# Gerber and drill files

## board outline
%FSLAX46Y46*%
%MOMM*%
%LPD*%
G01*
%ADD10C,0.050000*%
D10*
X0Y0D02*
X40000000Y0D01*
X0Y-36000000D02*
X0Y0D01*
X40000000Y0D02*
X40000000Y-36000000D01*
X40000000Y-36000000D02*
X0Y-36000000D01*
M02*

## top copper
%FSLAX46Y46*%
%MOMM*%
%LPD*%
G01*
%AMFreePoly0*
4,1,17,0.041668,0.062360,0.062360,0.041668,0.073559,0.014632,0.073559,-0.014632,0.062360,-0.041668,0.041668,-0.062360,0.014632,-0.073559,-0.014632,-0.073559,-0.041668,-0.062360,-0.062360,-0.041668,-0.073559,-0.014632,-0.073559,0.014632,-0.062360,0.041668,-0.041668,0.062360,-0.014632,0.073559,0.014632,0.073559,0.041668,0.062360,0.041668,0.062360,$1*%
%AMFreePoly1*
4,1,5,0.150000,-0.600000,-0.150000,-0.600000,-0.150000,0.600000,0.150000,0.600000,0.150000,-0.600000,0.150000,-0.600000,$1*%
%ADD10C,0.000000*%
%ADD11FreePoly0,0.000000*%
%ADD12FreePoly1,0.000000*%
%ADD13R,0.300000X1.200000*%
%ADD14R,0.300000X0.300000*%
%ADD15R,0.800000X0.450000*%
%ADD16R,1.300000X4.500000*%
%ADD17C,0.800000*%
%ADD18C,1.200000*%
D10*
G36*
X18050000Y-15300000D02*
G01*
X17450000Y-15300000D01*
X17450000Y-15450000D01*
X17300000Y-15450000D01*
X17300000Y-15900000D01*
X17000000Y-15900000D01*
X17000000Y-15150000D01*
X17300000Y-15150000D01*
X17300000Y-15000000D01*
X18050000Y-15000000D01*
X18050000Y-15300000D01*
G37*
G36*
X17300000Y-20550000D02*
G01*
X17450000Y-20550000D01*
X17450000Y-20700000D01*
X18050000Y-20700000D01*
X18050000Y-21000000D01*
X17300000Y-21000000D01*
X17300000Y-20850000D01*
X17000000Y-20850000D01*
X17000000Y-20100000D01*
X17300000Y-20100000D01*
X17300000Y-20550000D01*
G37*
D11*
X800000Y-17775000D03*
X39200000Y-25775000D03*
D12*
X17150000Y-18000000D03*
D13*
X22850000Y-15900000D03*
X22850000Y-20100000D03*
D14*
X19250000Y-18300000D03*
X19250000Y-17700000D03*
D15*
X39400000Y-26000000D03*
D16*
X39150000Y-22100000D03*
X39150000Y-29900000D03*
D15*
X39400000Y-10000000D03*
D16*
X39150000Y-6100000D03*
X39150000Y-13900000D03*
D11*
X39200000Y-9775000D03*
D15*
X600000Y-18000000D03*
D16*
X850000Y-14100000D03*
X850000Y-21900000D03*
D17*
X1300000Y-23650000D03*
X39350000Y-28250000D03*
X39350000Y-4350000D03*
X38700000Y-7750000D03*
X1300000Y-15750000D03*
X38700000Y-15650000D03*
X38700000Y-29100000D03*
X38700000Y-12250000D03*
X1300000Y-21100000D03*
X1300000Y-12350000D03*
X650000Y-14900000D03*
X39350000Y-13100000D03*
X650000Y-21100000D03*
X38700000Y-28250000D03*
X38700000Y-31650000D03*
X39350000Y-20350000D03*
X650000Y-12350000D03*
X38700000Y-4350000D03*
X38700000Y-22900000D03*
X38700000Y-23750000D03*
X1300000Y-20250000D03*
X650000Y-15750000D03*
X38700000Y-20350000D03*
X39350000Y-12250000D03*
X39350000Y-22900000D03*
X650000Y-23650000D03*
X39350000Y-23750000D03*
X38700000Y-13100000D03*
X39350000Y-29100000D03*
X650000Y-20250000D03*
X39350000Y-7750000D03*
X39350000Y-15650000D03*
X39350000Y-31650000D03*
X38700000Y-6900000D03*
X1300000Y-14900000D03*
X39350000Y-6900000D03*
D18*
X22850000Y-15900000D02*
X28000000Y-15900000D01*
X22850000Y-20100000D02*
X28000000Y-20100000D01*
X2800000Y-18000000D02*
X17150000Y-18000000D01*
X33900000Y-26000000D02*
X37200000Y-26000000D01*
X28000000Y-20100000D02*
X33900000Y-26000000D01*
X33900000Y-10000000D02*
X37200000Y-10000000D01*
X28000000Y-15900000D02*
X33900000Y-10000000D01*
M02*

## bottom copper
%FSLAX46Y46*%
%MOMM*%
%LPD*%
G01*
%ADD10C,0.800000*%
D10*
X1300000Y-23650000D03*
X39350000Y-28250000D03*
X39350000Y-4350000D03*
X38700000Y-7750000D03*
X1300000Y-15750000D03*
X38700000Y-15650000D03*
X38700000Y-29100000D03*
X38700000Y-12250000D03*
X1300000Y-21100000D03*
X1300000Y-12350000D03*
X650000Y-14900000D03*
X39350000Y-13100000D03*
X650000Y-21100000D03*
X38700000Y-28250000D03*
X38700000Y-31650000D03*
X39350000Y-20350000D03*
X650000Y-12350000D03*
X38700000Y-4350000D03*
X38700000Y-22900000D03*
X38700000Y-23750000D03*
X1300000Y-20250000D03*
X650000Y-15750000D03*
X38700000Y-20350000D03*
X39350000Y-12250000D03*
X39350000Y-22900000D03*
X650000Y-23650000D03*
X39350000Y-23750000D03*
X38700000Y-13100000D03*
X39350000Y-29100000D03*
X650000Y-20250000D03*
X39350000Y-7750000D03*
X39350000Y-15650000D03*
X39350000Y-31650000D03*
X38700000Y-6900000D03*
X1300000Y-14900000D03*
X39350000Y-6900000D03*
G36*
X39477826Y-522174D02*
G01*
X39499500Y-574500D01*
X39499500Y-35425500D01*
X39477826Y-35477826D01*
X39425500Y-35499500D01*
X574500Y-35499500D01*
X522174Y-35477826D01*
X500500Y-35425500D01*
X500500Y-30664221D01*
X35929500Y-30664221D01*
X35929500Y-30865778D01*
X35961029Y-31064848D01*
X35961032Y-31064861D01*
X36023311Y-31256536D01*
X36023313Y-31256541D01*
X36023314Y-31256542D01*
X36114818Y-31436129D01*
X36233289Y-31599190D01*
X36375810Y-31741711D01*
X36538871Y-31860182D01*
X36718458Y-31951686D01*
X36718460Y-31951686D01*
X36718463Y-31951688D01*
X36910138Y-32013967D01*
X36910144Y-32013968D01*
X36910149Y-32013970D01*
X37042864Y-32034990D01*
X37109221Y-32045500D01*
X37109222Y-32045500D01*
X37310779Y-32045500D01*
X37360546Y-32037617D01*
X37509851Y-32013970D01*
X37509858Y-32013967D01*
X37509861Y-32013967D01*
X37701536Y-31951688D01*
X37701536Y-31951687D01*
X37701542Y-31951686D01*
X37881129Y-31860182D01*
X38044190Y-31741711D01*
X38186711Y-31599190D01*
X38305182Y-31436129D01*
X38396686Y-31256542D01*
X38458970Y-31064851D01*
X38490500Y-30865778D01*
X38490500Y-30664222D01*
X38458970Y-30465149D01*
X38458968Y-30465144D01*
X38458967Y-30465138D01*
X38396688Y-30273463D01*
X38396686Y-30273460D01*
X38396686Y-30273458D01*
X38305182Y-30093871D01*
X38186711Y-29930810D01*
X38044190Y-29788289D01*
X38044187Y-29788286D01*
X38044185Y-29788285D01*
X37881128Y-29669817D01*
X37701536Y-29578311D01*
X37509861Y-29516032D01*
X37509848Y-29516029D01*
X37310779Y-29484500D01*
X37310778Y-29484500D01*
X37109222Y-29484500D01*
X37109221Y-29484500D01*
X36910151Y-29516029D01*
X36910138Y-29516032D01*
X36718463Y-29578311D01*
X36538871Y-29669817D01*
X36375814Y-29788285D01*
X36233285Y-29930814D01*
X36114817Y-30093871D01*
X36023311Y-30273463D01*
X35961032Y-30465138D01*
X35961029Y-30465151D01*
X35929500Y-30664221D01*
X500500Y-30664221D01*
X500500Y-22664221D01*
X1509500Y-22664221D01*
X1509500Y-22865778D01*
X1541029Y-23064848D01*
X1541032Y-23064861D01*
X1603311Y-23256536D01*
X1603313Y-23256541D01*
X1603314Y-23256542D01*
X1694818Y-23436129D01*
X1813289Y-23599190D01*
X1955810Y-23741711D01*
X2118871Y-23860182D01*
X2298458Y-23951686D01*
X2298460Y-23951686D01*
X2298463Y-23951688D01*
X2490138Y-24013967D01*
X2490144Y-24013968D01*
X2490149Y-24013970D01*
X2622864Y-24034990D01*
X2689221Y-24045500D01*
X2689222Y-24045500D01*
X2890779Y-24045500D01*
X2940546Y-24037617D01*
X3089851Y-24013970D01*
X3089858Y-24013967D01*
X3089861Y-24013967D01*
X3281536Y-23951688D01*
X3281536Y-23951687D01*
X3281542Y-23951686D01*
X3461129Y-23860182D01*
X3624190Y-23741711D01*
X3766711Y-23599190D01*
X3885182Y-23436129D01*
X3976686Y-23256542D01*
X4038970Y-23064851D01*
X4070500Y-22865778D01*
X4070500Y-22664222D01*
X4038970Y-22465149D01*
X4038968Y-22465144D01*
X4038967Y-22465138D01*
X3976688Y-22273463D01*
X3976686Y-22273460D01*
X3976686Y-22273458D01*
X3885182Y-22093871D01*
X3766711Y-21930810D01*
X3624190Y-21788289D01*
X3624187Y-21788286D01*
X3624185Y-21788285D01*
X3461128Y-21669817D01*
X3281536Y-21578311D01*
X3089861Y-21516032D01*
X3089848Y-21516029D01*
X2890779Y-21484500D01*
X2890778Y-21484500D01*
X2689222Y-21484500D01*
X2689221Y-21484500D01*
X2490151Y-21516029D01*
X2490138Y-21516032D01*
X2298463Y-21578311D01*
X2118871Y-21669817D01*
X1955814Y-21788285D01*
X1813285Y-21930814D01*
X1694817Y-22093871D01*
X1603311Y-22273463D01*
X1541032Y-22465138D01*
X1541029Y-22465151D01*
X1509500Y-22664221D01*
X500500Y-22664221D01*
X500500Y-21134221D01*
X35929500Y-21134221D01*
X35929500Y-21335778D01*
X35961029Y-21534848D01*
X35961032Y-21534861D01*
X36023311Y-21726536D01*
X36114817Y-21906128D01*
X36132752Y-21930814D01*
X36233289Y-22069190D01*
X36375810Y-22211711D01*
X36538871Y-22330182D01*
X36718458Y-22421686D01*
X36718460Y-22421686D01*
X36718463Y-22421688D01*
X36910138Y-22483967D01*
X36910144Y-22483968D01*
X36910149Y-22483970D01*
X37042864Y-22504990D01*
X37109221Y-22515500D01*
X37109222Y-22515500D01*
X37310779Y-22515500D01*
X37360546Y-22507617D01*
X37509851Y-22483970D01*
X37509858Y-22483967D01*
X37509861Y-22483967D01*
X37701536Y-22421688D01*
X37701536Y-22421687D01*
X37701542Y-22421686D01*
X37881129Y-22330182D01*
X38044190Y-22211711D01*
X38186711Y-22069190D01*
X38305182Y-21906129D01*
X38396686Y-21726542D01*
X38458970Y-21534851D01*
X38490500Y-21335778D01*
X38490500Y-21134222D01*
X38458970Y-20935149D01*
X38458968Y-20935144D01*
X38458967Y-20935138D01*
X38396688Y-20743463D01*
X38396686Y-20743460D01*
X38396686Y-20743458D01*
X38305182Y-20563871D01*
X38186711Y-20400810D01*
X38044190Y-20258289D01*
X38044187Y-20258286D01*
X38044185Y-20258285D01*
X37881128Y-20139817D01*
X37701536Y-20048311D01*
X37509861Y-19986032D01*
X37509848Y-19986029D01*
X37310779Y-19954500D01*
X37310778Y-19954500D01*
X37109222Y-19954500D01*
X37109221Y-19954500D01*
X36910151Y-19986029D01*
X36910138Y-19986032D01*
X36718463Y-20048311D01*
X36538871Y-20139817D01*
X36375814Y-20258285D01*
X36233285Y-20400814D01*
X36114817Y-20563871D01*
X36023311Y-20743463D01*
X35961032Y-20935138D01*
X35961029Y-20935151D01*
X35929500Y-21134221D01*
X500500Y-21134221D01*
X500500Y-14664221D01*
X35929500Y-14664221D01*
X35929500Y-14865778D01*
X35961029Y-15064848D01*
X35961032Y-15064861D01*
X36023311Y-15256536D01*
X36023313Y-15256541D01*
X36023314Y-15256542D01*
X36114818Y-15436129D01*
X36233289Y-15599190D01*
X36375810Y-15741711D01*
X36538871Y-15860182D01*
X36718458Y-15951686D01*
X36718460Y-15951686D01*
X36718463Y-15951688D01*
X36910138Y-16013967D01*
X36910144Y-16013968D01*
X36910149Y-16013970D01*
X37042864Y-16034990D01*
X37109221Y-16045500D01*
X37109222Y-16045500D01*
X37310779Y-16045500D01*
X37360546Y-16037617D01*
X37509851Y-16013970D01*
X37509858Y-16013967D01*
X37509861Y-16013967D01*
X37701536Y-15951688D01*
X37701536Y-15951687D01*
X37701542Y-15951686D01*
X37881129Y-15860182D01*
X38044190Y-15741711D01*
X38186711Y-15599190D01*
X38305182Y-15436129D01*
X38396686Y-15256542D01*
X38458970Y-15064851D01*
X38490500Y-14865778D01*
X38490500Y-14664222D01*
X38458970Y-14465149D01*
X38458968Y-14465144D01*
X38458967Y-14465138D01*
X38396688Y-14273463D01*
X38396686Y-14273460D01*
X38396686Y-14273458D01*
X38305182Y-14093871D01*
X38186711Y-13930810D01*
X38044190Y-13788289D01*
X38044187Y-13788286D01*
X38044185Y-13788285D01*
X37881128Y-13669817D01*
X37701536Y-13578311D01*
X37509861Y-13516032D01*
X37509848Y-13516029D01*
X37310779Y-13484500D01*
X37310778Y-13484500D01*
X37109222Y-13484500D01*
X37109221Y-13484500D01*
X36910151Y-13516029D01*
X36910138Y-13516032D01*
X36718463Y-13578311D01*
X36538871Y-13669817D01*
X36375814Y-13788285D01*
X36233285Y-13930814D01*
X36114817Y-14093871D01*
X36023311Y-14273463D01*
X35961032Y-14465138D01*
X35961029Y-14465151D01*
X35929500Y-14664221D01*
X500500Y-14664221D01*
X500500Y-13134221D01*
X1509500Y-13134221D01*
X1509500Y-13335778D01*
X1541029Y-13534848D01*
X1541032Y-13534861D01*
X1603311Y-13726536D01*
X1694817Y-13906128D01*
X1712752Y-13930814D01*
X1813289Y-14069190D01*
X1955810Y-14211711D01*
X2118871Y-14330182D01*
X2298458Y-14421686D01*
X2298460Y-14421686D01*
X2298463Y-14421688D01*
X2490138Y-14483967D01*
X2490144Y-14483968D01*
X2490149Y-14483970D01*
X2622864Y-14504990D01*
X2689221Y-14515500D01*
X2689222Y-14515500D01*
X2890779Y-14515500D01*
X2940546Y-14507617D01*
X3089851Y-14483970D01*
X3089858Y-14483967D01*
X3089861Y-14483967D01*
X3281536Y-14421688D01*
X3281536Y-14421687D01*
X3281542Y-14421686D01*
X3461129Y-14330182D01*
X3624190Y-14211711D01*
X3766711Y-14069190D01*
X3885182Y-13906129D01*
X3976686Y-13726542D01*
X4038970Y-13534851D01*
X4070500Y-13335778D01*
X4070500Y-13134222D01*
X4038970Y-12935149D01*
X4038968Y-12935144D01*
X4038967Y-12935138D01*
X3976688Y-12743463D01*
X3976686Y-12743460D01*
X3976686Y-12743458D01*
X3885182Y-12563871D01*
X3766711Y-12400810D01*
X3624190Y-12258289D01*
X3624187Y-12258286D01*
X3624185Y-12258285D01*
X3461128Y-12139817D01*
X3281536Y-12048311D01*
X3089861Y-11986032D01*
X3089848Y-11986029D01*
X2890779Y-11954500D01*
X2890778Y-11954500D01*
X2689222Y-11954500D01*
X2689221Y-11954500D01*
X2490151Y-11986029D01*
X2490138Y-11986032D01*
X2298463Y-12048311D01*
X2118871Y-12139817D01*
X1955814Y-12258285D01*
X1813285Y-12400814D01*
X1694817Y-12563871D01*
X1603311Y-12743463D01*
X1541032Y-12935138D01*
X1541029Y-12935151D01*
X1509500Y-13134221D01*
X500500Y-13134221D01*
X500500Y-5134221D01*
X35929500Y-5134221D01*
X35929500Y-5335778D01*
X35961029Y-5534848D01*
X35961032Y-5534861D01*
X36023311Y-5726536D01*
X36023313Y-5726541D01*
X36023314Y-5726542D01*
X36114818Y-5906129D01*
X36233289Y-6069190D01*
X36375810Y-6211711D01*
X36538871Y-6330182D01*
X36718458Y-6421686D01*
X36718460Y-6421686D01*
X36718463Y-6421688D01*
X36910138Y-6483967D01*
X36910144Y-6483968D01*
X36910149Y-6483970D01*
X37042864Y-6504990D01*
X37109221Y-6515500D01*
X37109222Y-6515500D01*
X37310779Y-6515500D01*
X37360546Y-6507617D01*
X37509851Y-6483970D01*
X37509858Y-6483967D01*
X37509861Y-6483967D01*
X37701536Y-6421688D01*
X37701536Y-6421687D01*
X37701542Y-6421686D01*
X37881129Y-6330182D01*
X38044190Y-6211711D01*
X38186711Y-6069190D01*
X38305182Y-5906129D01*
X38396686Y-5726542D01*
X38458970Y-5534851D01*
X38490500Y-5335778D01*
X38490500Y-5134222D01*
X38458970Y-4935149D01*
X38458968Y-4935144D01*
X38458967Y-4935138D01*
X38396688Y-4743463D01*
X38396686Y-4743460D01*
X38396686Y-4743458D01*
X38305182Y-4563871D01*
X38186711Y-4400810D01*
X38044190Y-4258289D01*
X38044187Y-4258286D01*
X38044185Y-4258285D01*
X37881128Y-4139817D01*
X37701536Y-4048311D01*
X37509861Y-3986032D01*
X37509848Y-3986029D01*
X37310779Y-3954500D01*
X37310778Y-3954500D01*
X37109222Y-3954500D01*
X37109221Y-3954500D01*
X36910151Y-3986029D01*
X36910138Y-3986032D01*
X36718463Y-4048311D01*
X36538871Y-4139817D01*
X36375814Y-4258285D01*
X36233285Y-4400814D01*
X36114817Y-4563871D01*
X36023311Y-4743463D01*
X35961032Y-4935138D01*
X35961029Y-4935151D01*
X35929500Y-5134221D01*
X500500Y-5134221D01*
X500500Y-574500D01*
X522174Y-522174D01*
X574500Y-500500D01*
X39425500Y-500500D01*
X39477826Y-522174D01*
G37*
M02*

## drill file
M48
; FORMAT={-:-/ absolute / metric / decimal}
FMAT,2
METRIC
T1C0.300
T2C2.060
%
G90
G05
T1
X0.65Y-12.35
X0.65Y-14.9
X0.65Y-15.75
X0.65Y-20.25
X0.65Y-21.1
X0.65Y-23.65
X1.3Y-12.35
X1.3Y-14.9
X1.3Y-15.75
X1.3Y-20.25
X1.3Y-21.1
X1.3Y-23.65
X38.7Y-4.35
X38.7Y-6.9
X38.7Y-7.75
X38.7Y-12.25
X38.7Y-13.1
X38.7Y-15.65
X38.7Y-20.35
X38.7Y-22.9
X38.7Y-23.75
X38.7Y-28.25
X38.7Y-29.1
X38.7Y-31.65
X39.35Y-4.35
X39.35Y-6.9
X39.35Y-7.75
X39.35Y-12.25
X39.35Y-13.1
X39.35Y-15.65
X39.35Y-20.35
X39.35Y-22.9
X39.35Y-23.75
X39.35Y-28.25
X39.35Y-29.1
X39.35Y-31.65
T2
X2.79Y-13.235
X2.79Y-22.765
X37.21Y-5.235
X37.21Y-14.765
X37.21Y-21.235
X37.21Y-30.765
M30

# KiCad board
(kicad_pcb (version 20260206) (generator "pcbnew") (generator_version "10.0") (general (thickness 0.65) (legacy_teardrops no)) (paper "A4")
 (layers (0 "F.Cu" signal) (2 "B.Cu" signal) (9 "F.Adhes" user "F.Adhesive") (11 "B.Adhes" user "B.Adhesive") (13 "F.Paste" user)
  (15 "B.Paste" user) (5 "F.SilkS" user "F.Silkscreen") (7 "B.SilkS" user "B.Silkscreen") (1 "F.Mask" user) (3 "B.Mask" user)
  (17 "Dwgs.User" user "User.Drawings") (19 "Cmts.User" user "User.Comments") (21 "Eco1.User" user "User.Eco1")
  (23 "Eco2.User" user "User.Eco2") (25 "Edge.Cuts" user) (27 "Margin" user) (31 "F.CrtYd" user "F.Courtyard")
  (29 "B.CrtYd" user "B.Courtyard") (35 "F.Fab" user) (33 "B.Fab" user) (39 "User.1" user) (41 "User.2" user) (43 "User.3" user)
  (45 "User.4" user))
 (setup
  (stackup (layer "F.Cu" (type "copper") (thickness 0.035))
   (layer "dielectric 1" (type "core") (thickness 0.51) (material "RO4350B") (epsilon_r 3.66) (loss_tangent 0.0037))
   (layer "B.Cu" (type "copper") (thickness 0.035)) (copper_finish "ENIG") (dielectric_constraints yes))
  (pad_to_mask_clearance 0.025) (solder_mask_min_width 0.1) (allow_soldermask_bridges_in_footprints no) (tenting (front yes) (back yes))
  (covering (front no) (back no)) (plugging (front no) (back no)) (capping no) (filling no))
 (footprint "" (layer "F.Cu") (at 0 0)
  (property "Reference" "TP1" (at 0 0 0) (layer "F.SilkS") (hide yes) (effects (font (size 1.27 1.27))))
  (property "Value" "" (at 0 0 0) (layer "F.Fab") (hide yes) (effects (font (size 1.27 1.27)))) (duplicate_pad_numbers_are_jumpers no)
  (pad "1" smd custom (at 0.8 17.775) (size 0.15 0.15) (layers "F.Cu" "F.Mask") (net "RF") (options (clearance outline) (anchor circle))
   (primitives)))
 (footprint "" (layer "F.Cu") (at 0 0)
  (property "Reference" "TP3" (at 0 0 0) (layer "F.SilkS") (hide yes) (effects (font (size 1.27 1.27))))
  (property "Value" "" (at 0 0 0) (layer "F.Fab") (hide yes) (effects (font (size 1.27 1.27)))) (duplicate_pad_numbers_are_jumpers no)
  (pad "1" smd custom (at 39.2 25.775) (size 0.15 0.15) (layers "F.Cu" "F.Mask") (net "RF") (options (clearance outline) (anchor circle))
   (primitives)))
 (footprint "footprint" (layer "F.Cu") (at 20 18)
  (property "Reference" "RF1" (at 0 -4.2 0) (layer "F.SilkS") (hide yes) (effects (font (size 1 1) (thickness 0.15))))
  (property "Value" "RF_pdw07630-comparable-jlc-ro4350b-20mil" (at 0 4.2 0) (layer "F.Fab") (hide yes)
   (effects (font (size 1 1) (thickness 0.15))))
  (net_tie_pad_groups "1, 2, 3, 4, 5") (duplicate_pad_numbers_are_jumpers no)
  (fp_poly
   (pts (xy -2.7 -2.1) (xy -2.7 -2.55) (xy -2.55 -2.55) (xy -2.55 -2.7) (xy -1.95 -2.7) (xy -1.95 -3) (xy -2.7 -3) (xy -2.7 -2.85)
    (xy -3 -2.85) (xy -3 -2.1))
   (stroke (width 0) (type solid)) (fill yes) (layer "F.Cu"))
  (fp_poly
   (pts (xy -2.7 2.85) (xy -2.7 3) (xy -1.95 3) (xy -1.95 2.7) (xy -2.55 2.7) (xy -2.55 2.55) (xy -2.7 2.55) (xy -2.7 2.1) (xy -3 2.1)
    (xy -3 2.85))
   (stroke (width 0) (type solid)) (fill yes) (layer "F.Cu"))
  (pad "1" smd custom (at -2.85 0) (size 0.3 1.2) (layers "F.Cu") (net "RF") (options (clearance outline) (anchor rect)) (primitives))
  (pad "2" smd rect (at 2.85 -2.1) (size 0.3 1.2) (layers "F.Cu") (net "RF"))
  (pad "3" smd rect (at 2.85 2.1) (size 0.3 1.2) (layers "F.Cu") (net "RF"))
  (pad "4" smd rect (at -0.75 0.3) (size 0.3 0.3) (layers "F.Cu") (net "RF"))
  (pad "5" smd rect (at -0.75 -0.3) (size 0.3 0.3) (layers "F.Cu") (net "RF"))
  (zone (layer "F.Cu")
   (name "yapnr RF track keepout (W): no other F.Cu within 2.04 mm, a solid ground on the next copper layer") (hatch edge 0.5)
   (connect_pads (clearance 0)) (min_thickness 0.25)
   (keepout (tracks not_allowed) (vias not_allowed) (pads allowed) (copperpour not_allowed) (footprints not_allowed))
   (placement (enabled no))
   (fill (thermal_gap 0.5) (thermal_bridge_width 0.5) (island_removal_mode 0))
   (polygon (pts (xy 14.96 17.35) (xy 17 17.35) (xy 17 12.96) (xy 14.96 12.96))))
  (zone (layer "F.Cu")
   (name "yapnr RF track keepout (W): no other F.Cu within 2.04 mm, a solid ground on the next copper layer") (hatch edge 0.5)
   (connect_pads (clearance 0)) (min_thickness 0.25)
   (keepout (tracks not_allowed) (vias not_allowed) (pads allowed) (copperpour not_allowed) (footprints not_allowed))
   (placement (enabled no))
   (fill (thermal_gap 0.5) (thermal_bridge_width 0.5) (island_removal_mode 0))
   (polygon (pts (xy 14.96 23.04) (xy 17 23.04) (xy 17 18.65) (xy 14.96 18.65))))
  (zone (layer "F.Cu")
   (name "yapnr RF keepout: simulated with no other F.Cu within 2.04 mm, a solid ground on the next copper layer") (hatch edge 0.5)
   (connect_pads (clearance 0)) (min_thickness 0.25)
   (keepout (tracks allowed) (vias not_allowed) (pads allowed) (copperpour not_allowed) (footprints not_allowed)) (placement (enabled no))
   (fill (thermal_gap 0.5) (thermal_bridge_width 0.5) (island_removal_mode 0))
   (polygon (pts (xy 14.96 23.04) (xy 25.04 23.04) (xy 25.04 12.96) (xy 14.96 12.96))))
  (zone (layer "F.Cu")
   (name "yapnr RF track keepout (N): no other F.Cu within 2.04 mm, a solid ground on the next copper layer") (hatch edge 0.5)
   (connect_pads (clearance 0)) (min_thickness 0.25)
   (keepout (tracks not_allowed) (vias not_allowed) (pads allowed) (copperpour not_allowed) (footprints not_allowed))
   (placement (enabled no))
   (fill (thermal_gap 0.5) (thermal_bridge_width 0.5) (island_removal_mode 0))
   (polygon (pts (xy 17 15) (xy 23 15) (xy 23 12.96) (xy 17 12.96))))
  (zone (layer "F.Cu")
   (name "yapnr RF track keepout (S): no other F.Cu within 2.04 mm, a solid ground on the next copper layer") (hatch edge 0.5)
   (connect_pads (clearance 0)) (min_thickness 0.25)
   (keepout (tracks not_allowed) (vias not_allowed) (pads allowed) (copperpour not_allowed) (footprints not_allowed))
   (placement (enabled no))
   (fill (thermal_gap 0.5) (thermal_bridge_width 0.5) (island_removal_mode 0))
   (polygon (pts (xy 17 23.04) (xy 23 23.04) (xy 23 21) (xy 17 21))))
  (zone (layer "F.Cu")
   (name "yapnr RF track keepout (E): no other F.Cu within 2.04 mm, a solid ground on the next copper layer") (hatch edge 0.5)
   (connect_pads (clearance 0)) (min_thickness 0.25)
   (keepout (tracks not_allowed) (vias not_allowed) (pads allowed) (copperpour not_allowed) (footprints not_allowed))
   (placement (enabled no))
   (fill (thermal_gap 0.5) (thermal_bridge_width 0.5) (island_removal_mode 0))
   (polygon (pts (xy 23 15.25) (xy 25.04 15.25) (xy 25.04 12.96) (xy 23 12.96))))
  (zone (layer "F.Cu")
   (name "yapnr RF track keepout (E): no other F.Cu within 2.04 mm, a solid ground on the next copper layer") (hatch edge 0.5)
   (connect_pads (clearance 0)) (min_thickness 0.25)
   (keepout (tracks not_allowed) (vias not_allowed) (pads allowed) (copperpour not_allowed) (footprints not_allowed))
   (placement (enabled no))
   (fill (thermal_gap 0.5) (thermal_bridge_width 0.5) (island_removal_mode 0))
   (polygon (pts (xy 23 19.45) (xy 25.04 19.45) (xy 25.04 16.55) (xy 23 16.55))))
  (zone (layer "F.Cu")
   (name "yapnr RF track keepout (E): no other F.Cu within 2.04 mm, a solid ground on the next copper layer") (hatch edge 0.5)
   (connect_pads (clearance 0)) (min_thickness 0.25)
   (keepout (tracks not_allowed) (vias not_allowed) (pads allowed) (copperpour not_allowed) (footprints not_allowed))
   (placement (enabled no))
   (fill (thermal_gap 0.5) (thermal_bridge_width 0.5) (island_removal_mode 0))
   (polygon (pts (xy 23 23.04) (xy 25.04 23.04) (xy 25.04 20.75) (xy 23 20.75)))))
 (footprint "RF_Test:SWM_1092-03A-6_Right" (layer "F.Cu") (at 40 26)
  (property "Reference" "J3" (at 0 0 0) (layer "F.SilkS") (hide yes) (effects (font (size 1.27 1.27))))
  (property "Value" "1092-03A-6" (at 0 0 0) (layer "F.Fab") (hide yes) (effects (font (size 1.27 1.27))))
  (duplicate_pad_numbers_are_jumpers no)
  (pad "" np_thru_hole circle (at -2.79 -4.765) (size 2.06 2.06) (drill 2.06) (layers "*.Cu" "*.Mask"))
  (pad "" np_thru_hole circle (at -2.79 4.765) (size 2.06 2.06) (drill 2.06) (layers "*.Cu" "*.Mask"))
  (pad "1" smd rect (at -0.6 0) (size 0.8 0.45) (layers "F.Cu" "F.Mask") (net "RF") (thermal_bridge_angle 45))
  (pad "2" smd rect (at -0.85 -3.9) (size 1.3 4.5) (layers "F.Cu" "F.Mask") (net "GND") (thermal_bridge_angle 45))
  (pad "3" smd rect (at -0.85 3.9) (size 1.3 4.5) (layers "F.Cu" "F.Mask") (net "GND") (thermal_bridge_angle 45)))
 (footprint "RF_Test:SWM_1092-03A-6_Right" (layer "F.Cu") (at 40 10)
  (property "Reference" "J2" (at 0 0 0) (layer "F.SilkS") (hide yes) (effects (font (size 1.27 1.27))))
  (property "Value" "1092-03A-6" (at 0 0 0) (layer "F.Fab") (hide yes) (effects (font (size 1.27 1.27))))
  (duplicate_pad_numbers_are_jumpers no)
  (pad "" np_thru_hole circle (at -2.79 -4.765) (size 2.06 2.06) (drill 2.06) (layers "*.Cu" "*.Mask"))
  (pad "" np_thru_hole circle (at -2.79 4.765) (size 2.06 2.06) (drill 2.06) (layers "*.Cu" "*.Mask"))
  (pad "1" smd rect (at -0.6 0) (size 0.8 0.45) (layers "F.Cu" "F.Mask") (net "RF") (thermal_bridge_angle 45))
  (pad "2" smd rect (at -0.85 -3.9) (size 1.3 4.5) (layers "F.Cu" "F.Mask") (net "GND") (thermal_bridge_angle 45))
  (pad "3" smd rect (at -0.85 3.9) (size 1.3 4.5) (layers "F.Cu" "F.Mask") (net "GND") (thermal_bridge_angle 45)))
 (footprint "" (layer "F.Cu") (at 0 0)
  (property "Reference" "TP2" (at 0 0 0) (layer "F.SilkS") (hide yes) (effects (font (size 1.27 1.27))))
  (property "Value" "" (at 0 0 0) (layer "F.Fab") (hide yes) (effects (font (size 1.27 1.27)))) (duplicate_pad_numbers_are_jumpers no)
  (pad "1" smd custom (at 39.2 9.775) (size 0.15 0.15) (layers "F.Cu" "F.Mask") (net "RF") (options (clearance outline) (anchor circle))
   (primitives)))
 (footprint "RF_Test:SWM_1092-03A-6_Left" (layer "F.Cu") (at 0 18)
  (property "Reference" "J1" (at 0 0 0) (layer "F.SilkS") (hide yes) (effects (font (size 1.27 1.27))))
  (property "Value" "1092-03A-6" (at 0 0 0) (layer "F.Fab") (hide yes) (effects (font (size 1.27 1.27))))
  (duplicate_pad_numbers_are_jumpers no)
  (pad "" np_thru_hole circle (at 2.79 -4.765) (size 2.06 2.06) (drill 2.06) (layers "*.Cu" "*.Mask"))
  (pad "" np_thru_hole circle (at 2.79 4.765) (size 2.06 2.06) (drill 2.06) (layers "*.Cu" "*.Mask"))
  (pad "1" smd rect (at 0.6 0) (size 0.8 0.45) (layers "F.Cu" "F.Mask") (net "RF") (thermal_bridge_angle 45))
  (pad "2" smd rect (at 0.85 -3.9) (size 1.3 4.5) (layers "F.Cu" "F.Mask") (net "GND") (thermal_bridge_angle 45))
  (pad "3" smd rect (at 0.85 3.9) (size 1.3 4.5) (layers "F.Cu" "F.Mask") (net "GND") (thermal_bridge_angle 45)))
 (gr_line (start 0 0) (end 40 0) (stroke (width 0.05) (type default)) (layer "Edge.Cuts"))
 (gr_line (start 0 36) (end 0 0) (stroke (width 0.05) (type default)) (layer "Edge.Cuts"))
 (gr_line (start 40 0) (end 40 36) (stroke (width 0.05) (type default)) (layer "Edge.Cuts"))
 (gr_line (start 40 36) (end 0 36) (stroke (width 0.05) (type default)) (layer "Edge.Cuts"))
 (via (at 1.3 23.65) (size 0.8) (drill 0.3) (layers "F.Cu" "B.Cu") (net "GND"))
 (via (at 39.35 28.25) (size 0.8) (drill 0.3) (layers "F.Cu" "B.Cu") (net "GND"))
 (via (at 39.35 4.35) (size 0.8) (drill 0.3) (layers "F.Cu" "B.Cu") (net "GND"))
 (via (at 38.7 7.75) (size 0.8) (drill 0.3) (layers "F.Cu" "B.Cu") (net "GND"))
 (via (at 1.3 15.75) (size 0.8) (drill 0.3) (layers "F.Cu" "B.Cu") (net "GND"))
 (via (at 38.7 15.65) (size 0.8) (drill 0.3) (layers "F.Cu" "B.Cu") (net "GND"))
 (via (at 38.7 29.1) (size 0.8) (drill 0.3) (layers "F.Cu" "B.Cu") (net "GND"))
 (via (at 38.7 12.25) (size 0.8) (drill 0.3) (layers "F.Cu" "B.Cu") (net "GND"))
 (via (at 1.3 21.1) (size 0.8) (drill 0.3) (layers "F.Cu" "B.Cu") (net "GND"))
 (via (at 1.3 12.35) (size 0.8) (drill 0.3) (layers "F.Cu" "B.Cu") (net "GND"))
 (via (at 0.65 14.9) (size 0.8) (drill 0.3) (layers "F.Cu" "B.Cu") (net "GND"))
 (via (at 39.35 13.1) (size 0.8) (drill 0.3) (layers "F.Cu" "B.Cu") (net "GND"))
 (via (at 0.65 21.1) (size 0.8) (drill 0.3) (layers "F.Cu" "B.Cu") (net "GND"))
 (via (at 38.7 28.25) (size 0.8) (drill 0.3) (layers "F.Cu" "B.Cu") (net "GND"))
 (via (at 38.7 31.65) (size 0.8) (drill 0.3) (layers "F.Cu" "B.Cu") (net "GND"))
 (via (at 39.35 20.35) (size 0.8) (drill 0.3) (layers "F.Cu" "B.Cu") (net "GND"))
 (via (at 0.65 12.35) (size 0.8) (drill 0.3) (layers "F.Cu" "B.Cu") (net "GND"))
 (via (at 38.7 4.35) (size 0.8) (drill 0.3) (layers "F.Cu" "B.Cu") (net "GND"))
 (via (at 38.7 22.9) (size 0.8) (drill 0.3) (layers "F.Cu" "B.Cu") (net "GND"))
 (via (at 38.7 23.75) (size 0.8) (drill 0.3) (layers "F.Cu" "B.Cu") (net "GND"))
 (via (at 1.3 20.25) (size 0.8) (drill 0.3) (layers "F.Cu" "B.Cu") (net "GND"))
 (via (at 0.65 15.75) (size 0.8) (drill 0.3) (layers "F.Cu" "B.Cu") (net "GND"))
 (via (at 38.7 20.35) (size 0.8) (drill 0.3) (layers "F.Cu" "B.Cu") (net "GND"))
 (via (at 39.35 12.25) (size 0.8) (drill 0.3) (layers "F.Cu" "B.Cu") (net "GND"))
 (via (at 39.35 22.9) (size 0.8) (drill 0.3) (layers "F.Cu" "B.Cu") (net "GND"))
 (via (at 0.65 23.65) (size 0.8) (drill 0.3) (layers "F.Cu" "B.Cu") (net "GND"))
 (via (at 39.35 23.75) (size 0.8) (drill 0.3) (layers "F.Cu" "B.Cu") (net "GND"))
 (via (at 38.7 13.1) (size 0.8) (drill 0.3) (layers "F.Cu" "B.Cu") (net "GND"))
 (via (at 39.35 29.1) (size 0.8) (drill 0.3) (layers "F.Cu" "B.Cu") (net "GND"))
 (via (at 0.65 20.25) (size 0.8) (drill 0.3) (layers "F.Cu" "B.Cu") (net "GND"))
 (via (at 39.35 7.75) (size 0.8) (drill 0.3) (layers "F.Cu" "B.Cu") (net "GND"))
 (via (at 39.35 15.65) (size 0.8) (drill 0.3) (layers "F.Cu" "B.Cu") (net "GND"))
 (via (at 39.35 31.65) (size 0.8) (drill 0.3) (layers "F.Cu" "B.Cu") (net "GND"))
 (via (at 38.7 6.9) (size 0.8) (drill 0.3) (layers "F.Cu" "B.Cu") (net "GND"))
 (via (at 1.3 14.9) (size 0.8) (drill 0.3) (layers "F.Cu" "B.Cu") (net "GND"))
 (via (at 39.35 6.9) (size 0.8) (drill 0.3) (layers "F.Cu" "B.Cu") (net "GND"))
 (segment (start 22.85 15.9) (end 28 15.9) (width 1.2) (layer "F.Cu") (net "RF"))
 (segment (start 22.85 20.1) (end 28 20.1) (width 1.2) (layer "F.Cu") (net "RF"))
 (segment (start 2.8 18) (end 17.15 18) (width 1.2) (layer "F.Cu") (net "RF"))
 (segment (start 33.9 26) (end 37.2 26) (width 1.2) (layer "F.Cu") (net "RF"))
 (segment (start 28 20.1) (end 33.9 26) (width 1.2) (layer "F.Cu") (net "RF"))
 (segment (start 33.9 10) (end 37.2 10) (width 1.2) (layer "F.Cu") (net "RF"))
 (segment (start 28 15.9) (end 33.9 10) (width 1.2) (layer "F.Cu") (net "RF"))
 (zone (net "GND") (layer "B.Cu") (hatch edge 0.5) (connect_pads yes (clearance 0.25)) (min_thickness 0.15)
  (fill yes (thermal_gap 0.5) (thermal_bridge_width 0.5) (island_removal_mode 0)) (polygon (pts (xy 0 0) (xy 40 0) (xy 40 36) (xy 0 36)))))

